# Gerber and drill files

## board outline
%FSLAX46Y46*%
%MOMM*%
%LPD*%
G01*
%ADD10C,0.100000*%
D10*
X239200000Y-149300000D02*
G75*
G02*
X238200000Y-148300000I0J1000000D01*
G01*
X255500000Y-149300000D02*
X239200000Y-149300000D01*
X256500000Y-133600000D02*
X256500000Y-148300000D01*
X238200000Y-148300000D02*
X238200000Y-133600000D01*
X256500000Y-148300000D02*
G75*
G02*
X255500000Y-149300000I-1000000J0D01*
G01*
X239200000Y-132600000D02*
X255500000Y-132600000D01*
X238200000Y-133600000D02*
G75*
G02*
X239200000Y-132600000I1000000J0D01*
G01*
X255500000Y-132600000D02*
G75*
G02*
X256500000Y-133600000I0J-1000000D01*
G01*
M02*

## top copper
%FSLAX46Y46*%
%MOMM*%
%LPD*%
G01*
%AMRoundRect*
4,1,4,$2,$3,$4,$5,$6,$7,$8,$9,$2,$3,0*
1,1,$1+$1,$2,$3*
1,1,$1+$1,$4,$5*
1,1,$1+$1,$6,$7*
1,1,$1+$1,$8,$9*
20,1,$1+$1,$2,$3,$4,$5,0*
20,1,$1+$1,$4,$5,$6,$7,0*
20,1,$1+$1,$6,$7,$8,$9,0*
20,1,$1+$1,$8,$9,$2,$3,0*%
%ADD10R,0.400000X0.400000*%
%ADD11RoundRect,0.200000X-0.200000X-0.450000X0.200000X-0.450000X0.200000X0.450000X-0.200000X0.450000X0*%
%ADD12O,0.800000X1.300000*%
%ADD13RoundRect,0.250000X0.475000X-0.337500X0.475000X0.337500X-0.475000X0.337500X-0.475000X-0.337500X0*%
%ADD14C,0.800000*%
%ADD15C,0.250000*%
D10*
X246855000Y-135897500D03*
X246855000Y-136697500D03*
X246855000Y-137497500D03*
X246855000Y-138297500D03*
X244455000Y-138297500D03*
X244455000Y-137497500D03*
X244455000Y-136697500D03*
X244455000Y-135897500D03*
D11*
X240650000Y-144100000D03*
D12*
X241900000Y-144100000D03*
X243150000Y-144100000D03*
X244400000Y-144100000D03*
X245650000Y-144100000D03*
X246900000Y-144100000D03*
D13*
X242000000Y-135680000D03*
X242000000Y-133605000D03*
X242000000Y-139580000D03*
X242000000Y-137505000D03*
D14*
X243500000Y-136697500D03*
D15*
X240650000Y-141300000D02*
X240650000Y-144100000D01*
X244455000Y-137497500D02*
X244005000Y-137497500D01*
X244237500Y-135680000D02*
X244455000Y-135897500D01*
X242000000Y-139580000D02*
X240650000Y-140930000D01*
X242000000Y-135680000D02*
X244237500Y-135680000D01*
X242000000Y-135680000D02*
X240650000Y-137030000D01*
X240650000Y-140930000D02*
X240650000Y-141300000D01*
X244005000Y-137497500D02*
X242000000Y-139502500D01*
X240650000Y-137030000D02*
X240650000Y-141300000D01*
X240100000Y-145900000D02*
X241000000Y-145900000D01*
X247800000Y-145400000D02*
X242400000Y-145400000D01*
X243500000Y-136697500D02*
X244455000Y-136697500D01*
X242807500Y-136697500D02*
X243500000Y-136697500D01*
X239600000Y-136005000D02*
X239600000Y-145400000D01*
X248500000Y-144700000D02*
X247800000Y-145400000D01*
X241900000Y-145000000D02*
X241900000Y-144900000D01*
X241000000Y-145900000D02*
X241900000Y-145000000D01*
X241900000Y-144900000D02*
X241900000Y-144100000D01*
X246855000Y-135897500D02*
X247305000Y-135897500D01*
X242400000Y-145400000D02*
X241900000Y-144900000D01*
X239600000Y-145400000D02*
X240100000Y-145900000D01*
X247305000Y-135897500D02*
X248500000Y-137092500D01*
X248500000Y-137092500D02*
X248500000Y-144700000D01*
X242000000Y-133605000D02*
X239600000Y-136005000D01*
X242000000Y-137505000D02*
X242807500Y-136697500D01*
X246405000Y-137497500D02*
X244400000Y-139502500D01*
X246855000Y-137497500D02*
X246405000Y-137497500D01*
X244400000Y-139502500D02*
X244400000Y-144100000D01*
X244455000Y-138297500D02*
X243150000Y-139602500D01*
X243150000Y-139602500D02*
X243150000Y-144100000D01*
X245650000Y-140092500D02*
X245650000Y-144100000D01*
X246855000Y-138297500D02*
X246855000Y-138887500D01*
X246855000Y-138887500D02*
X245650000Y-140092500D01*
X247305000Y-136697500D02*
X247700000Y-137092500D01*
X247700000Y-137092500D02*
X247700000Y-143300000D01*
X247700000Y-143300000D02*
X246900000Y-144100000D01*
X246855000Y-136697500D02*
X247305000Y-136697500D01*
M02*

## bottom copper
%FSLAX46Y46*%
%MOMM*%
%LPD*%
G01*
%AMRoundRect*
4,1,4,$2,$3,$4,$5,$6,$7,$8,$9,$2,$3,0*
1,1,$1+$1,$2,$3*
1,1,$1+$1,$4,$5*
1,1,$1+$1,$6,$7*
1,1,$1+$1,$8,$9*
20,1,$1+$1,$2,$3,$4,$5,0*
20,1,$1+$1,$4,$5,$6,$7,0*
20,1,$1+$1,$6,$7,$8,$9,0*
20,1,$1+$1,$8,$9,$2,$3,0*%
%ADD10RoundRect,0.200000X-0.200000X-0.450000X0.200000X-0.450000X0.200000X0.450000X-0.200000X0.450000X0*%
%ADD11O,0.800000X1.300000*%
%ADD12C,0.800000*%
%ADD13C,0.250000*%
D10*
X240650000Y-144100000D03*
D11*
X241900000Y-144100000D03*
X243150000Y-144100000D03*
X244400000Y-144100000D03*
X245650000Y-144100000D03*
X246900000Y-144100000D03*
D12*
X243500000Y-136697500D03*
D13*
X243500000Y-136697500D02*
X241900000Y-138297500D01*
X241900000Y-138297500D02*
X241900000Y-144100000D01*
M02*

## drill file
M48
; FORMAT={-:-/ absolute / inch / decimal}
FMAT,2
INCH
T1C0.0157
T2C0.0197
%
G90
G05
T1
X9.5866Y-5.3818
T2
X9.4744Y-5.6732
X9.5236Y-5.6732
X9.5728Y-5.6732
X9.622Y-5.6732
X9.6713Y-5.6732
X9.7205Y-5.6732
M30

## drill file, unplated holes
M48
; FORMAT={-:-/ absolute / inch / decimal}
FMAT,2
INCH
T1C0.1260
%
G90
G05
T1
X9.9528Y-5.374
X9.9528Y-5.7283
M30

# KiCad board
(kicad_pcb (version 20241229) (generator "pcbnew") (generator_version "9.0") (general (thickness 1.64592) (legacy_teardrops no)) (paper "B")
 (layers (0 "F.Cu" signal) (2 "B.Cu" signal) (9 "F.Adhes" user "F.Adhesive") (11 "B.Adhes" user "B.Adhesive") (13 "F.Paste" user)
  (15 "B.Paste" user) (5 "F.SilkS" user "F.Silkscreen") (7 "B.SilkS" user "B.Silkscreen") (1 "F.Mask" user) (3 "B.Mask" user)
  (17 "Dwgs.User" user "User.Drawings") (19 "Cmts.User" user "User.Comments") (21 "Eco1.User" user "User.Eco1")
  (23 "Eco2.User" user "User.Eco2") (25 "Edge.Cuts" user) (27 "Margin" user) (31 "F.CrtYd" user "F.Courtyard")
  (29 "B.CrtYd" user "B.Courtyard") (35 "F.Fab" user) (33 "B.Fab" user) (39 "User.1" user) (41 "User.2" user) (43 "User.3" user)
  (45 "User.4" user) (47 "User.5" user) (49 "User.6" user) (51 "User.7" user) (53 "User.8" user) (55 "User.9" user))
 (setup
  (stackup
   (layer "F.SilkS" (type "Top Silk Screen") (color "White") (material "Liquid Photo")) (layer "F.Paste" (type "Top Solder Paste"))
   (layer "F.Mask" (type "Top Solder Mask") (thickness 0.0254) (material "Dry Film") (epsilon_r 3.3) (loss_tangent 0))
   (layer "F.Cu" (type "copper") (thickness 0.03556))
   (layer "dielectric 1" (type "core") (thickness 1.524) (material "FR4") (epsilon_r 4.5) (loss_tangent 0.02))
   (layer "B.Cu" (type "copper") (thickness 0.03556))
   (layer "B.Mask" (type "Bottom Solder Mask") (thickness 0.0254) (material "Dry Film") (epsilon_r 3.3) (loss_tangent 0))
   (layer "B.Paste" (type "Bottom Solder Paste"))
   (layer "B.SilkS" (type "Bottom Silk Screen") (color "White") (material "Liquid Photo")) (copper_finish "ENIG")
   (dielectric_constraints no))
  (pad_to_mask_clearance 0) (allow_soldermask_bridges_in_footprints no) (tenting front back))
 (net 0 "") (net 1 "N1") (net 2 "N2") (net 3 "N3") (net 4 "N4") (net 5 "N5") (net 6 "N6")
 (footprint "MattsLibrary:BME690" (layer "F.Cu") (at 245.655 137.0975)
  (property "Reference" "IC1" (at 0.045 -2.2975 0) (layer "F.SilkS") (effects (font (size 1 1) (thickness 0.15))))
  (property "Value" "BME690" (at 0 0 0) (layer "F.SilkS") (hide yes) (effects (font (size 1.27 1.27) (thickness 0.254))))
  (pad "1" smd rect (at 1.2 -1.2 90) (size 0.4 0.4) (layers "F.Cu" "F.Mask" "F.Paste") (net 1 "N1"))
  (pad "2" smd rect (at 1.2 -0.4 90) (size 0.4 0.4) (layers "F.Cu" "F.Mask" "F.Paste") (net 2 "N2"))
  (pad "3" smd rect (at 1.2 0.4 90) (size 0.4 0.4) (layers "F.Cu" "F.Mask" "F.Paste") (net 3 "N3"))
  (pad "4" smd rect (at 1.2 1.2 90) (size 0.4 0.4) (layers "F.Cu" "F.Mask" "F.Paste") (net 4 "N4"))
  (pad "5" smd rect (at -1.2 1.2 90) (size 0.4 0.4) (layers "F.Cu" "F.Mask" "F.Paste") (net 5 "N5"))
  (pad "6" smd rect (at -1.2 0.4 90) (size 0.4 0.4) (layers "F.Cu" "F.Mask" "F.Paste") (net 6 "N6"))
  (pad "7" smd rect (at -1.2 -0.4 90) (size 0.4 0.4) (layers "F.Cu" "F.Mask" "F.Paste") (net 1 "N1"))
  (pad "8" smd rect (at -1.2 -1.2 90) (size 0.4 0.4) (layers "F.Cu" "F.Mask" "F.Paste") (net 6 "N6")))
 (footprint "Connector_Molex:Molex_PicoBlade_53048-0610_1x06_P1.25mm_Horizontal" (layer "F.Cu") (at 240.65 144.1)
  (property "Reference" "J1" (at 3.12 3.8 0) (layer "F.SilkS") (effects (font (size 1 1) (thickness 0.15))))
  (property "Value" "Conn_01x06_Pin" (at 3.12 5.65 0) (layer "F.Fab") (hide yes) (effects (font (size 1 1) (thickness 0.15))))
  (pad "1" thru_hole roundrect (at 0 0) (size 0.8 1.3) (drill 0.5) (layers "*.Cu" "*.Mask") (remove_unused_layers no)
   (roundrect_rratio 0.25) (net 6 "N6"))
  (pad "2" thru_hole oval (at 1.25 0) (size 0.8 1.3) (drill 0.5) (layers "*.Cu" "*.Mask") (remove_unused_layers no) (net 1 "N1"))
  (pad "3" thru_hole oval (at 2.5 0) (size 0.8 1.3) (drill 0.5) (layers "*.Cu" "*.Mask") (remove_unused_layers no) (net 5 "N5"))
  (pad "4" thru_hole oval (at 3.75 0) (size 0.8 1.3) (drill 0.5) (layers "*.Cu" "*.Mask") (remove_unused_layers no) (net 3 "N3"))
  (pad "5" thru_hole oval (at 5 0) (size 0.8 1.3) (drill 0.5) (layers "*.Cu" "*.Mask") (remove_unused_layers no) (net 4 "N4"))
  (pad "6" thru_hole oval (at 6.25 0) (size 0.8 1.3) (drill 0.5) (layers "*.Cu" "*.Mask") (remove_unused_layers no) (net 2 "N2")))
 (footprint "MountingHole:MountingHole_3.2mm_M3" (layer "F.Cu") (at 252.8 136.5)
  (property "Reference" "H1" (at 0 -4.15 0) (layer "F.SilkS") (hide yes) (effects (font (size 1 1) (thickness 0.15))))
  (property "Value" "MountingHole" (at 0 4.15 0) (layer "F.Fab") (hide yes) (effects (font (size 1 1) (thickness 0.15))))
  (pad "" np_thru_hole circle (at 0 0) (size 3.2 3.2) (drill 3.2) (layers "*.Cu" "*.Mask")))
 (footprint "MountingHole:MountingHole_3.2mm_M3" (layer "F.Cu") (at 252.8 145.5)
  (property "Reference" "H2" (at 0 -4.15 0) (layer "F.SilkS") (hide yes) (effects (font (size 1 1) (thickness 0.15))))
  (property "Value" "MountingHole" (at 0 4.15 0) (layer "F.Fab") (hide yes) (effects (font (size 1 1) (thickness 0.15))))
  (pad "" np_thru_hole circle (at 0 0) (size 3.2 3.2) (drill 3.2) (layers "*.Cu" "*.Mask")))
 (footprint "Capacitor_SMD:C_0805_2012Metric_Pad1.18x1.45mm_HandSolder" (layer "F.Cu") (at 242 134.6425 90)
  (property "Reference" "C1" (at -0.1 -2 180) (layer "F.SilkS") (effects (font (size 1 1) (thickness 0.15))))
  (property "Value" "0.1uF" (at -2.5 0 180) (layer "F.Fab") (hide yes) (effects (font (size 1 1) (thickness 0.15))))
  (pad "1" smd roundrect (at -1.0375 0 90) (size 1.175 1.45) (layers "F.Cu" "F.Mask" "F.Paste") (roundrect_rratio 0.212766) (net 6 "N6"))
  (pad "2" smd roundrect (at 1.0375 0 90) (size 1.175 1.45) (layers "F.Cu" "F.Mask" "F.Paste") (roundrect_rratio 0.212766) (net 1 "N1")))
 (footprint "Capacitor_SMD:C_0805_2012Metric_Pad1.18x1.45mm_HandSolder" (layer "F.Cu") (at 242 138.5425 90)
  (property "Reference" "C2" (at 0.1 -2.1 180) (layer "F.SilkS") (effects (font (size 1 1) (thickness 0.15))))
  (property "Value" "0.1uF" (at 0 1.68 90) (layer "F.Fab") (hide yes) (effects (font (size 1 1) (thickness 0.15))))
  (pad "1" smd roundrect (at -1.0375 0 90) (size 1.175 1.45) (layers "F.Cu" "F.Mask" "F.Paste") (roundrect_rratio 0.212766) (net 6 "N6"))
  (pad "2" smd roundrect (at 1.0375 0 90) (size 1.175 1.45) (layers "F.Cu" "F.Mask" "F.Paste") (roundrect_rratio 0.212766) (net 1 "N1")))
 (gr_arc (start 239.2 149.3) (mid 238.492893 149.007107) (end 238.2 148.3) (stroke (width 0.1) (type default)) (layer "Edge.Cuts"))
 (gr_line (start 255.5 149.3) (end 239.2 149.3) (stroke (width 0.1) (type default)) (layer "Edge.Cuts"))
 (gr_line (start 256.5 133.6) (end 256.5 148.3) (stroke (width 0.1) (type default)) (layer "Edge.Cuts"))
 (gr_line (start 238.2 148.3) (end 238.2 133.6) (stroke (width 0.1) (type default)) (layer "Edge.Cuts"))
 (gr_arc (start 256.5 148.3) (mid 256.207107 149.007107) (end 255.5 149.3) (stroke (width 0.1) (type default)) (layer "Edge.Cuts"))
 (gr_line (start 239.2 132.6) (end 255.5 132.6) (stroke (width 0.1) (type default)) (layer "Edge.Cuts"))
 (gr_arc (start 238.2 133.6) (mid 238.492893 132.892893) (end 239.2 132.6) (stroke (width 0.1) (type default)) (layer "Edge.Cuts"))
 (gr_arc (start 255.5 132.6) (mid 256.207107 132.892893) (end 256.5 133.6) (stroke (width 0.1) (type default)) (layer "Edge.Cuts"))
 (segment (start 240.65 141.3) (end 240.65 144.1) (width 0.25) (layer "F.Cu") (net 6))
 (segment (start 244.455 137.4975) (end 244.005 137.4975) (width 0.25) (layer "F.Cu") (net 6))
 (segment (start 244.2375 135.68) (end 244.455 135.8975) (width 0.25) (layer "F.Cu") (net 6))
 (segment (start 242 139.58) (end 240.65 140.93) (width 0.25) (layer "F.Cu") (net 6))
 (segment (start 242 135.68) (end 244.2375 135.68) (width 0.25) (layer "F.Cu") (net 6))
 (segment (start 242 135.68) (end 240.65 137.03) (width 0.25) (layer "F.Cu") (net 6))
 (segment (start 240.65 140.93) (end 240.65 141.3) (width 0.25) (layer "F.Cu") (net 6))
 (segment (start 244.005 137.4975) (end 242 139.5025) (width 0.25) (layer "F.Cu") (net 6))
 (segment (start 240.65 137.03) (end 240.65 141.3) (width 0.25) (layer "F.Cu") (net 6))
 (segment (start 240.1 145.9) (end 241 145.9) (width 0.25) (layer "F.Cu") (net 1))
 (segment (start 247.8 145.4) (end 242.4 145.4) (width 0.25) (layer "F.Cu") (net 1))
 (segment (start 243.5 136.6975) (end 244.455 136.6975) (width 0.25) (layer "F.Cu") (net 1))
 (segment (start 242.8075 136.6975) (end 243.5 136.6975) (width 0.25) (layer "F.Cu") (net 1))
 (segment (start 239.6 136.005) (end 239.6 145.4) (width 0.25) (layer "F.Cu") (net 1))
 (segment (start 248.5 144.7) (end 247.8 145.4) (width 0.25) (layer "F.Cu") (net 1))
 (segment (start 241.9 145) (end 241.9 144.9) (width 0.25) (layer "F.Cu") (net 1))
 (segment (start 241 145.9) (end 241.9 145) (width 0.25) (layer "F.Cu") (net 1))
 (segment (start 241.9 144.9) (end 241.9 144.1) (width 0.25) (layer "F.Cu") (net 1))
 (segment (start 246.855 135.8975) (end 247.305 135.8975) (width 0.25) (layer "F.Cu") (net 1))
 (segment (start 242.4 145.4) (end 241.9 144.9) (width 0.25) (layer "F.Cu") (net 1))
 (segment (start 239.6 145.4) (end 240.1 145.9) (width 0.25) (layer "F.Cu") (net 1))
 (segment (start 247.305 135.8975) (end 248.5 137.0925) (width 0.25) (layer "F.Cu") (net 1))
 (segment (start 248.5 137.0925) (end 248.5 144.7) (width 0.25) (layer "F.Cu") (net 1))
 (segment (start 242 133.605) (end 239.6 136.005) (width 0.25) (layer "F.Cu") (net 1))
 (segment (start 242 137.505) (end 242.8075 136.6975) (width 0.25) (layer "F.Cu") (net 1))
 (via (at 243.5 136.6975) (size 0.8) (drill 0.4) (layers "F.Cu" "B.Cu") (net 1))
 (segment (start 243.5 136.6975) (end 241.9 138.2975) (width 0.25) (layer "B.Cu") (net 1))
 (segment (start 241.9 138.2975) (end 241.9 144.1) (width 0.25) (layer "B.Cu") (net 1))
 (segment (start 246.405 137.4975) (end 244.4 139.5025) (width 0.25) (layer "F.Cu") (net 3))
 (segment (start 246.855 137.4975) (end 246.405 137.4975) (width 0.25) (layer "F.Cu") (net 3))
 (segment (start 244.4 139.5025) (end 244.4 144.1) (width 0.25) (layer "F.Cu") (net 3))
 (segment (start 244.455 138.2975) (end 243.15 139.6025) (width 0.25) (layer "F.Cu") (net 5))
 (segment (start 243.15 139.6025) (end 243.15 144.1) (width 0.25) (layer "F.Cu") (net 5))
 (segment (start 245.65 140.0925) (end 245.65 144.1) (width 0.25) (layer "F.Cu") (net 4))
 (segment (start 246.855 138.2975) (end 246.855 138.8875) (width 0.25) (layer "F.Cu") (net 4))
 (segment (start 246.855 138.8875) (end 245.65 140.0925) (width 0.25) (layer "F.Cu") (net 4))
 (segment (start 247.305 136.6975) (end 247.7 137.0925) (width 0.25) (layer "F.Cu") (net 2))
 (segment (start 247.7 137.0925) (end 247.7 143.3) (width 0.25) (layer "F.Cu") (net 2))
 (segment (start 247.7 143.3) (end 246.9 144.1) (width 0.25) (layer "F.Cu") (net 2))
 (segment (start 246.855 136.6975) (end 247.305 136.6975) (width 0.25) (layer "F.Cu") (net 2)))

